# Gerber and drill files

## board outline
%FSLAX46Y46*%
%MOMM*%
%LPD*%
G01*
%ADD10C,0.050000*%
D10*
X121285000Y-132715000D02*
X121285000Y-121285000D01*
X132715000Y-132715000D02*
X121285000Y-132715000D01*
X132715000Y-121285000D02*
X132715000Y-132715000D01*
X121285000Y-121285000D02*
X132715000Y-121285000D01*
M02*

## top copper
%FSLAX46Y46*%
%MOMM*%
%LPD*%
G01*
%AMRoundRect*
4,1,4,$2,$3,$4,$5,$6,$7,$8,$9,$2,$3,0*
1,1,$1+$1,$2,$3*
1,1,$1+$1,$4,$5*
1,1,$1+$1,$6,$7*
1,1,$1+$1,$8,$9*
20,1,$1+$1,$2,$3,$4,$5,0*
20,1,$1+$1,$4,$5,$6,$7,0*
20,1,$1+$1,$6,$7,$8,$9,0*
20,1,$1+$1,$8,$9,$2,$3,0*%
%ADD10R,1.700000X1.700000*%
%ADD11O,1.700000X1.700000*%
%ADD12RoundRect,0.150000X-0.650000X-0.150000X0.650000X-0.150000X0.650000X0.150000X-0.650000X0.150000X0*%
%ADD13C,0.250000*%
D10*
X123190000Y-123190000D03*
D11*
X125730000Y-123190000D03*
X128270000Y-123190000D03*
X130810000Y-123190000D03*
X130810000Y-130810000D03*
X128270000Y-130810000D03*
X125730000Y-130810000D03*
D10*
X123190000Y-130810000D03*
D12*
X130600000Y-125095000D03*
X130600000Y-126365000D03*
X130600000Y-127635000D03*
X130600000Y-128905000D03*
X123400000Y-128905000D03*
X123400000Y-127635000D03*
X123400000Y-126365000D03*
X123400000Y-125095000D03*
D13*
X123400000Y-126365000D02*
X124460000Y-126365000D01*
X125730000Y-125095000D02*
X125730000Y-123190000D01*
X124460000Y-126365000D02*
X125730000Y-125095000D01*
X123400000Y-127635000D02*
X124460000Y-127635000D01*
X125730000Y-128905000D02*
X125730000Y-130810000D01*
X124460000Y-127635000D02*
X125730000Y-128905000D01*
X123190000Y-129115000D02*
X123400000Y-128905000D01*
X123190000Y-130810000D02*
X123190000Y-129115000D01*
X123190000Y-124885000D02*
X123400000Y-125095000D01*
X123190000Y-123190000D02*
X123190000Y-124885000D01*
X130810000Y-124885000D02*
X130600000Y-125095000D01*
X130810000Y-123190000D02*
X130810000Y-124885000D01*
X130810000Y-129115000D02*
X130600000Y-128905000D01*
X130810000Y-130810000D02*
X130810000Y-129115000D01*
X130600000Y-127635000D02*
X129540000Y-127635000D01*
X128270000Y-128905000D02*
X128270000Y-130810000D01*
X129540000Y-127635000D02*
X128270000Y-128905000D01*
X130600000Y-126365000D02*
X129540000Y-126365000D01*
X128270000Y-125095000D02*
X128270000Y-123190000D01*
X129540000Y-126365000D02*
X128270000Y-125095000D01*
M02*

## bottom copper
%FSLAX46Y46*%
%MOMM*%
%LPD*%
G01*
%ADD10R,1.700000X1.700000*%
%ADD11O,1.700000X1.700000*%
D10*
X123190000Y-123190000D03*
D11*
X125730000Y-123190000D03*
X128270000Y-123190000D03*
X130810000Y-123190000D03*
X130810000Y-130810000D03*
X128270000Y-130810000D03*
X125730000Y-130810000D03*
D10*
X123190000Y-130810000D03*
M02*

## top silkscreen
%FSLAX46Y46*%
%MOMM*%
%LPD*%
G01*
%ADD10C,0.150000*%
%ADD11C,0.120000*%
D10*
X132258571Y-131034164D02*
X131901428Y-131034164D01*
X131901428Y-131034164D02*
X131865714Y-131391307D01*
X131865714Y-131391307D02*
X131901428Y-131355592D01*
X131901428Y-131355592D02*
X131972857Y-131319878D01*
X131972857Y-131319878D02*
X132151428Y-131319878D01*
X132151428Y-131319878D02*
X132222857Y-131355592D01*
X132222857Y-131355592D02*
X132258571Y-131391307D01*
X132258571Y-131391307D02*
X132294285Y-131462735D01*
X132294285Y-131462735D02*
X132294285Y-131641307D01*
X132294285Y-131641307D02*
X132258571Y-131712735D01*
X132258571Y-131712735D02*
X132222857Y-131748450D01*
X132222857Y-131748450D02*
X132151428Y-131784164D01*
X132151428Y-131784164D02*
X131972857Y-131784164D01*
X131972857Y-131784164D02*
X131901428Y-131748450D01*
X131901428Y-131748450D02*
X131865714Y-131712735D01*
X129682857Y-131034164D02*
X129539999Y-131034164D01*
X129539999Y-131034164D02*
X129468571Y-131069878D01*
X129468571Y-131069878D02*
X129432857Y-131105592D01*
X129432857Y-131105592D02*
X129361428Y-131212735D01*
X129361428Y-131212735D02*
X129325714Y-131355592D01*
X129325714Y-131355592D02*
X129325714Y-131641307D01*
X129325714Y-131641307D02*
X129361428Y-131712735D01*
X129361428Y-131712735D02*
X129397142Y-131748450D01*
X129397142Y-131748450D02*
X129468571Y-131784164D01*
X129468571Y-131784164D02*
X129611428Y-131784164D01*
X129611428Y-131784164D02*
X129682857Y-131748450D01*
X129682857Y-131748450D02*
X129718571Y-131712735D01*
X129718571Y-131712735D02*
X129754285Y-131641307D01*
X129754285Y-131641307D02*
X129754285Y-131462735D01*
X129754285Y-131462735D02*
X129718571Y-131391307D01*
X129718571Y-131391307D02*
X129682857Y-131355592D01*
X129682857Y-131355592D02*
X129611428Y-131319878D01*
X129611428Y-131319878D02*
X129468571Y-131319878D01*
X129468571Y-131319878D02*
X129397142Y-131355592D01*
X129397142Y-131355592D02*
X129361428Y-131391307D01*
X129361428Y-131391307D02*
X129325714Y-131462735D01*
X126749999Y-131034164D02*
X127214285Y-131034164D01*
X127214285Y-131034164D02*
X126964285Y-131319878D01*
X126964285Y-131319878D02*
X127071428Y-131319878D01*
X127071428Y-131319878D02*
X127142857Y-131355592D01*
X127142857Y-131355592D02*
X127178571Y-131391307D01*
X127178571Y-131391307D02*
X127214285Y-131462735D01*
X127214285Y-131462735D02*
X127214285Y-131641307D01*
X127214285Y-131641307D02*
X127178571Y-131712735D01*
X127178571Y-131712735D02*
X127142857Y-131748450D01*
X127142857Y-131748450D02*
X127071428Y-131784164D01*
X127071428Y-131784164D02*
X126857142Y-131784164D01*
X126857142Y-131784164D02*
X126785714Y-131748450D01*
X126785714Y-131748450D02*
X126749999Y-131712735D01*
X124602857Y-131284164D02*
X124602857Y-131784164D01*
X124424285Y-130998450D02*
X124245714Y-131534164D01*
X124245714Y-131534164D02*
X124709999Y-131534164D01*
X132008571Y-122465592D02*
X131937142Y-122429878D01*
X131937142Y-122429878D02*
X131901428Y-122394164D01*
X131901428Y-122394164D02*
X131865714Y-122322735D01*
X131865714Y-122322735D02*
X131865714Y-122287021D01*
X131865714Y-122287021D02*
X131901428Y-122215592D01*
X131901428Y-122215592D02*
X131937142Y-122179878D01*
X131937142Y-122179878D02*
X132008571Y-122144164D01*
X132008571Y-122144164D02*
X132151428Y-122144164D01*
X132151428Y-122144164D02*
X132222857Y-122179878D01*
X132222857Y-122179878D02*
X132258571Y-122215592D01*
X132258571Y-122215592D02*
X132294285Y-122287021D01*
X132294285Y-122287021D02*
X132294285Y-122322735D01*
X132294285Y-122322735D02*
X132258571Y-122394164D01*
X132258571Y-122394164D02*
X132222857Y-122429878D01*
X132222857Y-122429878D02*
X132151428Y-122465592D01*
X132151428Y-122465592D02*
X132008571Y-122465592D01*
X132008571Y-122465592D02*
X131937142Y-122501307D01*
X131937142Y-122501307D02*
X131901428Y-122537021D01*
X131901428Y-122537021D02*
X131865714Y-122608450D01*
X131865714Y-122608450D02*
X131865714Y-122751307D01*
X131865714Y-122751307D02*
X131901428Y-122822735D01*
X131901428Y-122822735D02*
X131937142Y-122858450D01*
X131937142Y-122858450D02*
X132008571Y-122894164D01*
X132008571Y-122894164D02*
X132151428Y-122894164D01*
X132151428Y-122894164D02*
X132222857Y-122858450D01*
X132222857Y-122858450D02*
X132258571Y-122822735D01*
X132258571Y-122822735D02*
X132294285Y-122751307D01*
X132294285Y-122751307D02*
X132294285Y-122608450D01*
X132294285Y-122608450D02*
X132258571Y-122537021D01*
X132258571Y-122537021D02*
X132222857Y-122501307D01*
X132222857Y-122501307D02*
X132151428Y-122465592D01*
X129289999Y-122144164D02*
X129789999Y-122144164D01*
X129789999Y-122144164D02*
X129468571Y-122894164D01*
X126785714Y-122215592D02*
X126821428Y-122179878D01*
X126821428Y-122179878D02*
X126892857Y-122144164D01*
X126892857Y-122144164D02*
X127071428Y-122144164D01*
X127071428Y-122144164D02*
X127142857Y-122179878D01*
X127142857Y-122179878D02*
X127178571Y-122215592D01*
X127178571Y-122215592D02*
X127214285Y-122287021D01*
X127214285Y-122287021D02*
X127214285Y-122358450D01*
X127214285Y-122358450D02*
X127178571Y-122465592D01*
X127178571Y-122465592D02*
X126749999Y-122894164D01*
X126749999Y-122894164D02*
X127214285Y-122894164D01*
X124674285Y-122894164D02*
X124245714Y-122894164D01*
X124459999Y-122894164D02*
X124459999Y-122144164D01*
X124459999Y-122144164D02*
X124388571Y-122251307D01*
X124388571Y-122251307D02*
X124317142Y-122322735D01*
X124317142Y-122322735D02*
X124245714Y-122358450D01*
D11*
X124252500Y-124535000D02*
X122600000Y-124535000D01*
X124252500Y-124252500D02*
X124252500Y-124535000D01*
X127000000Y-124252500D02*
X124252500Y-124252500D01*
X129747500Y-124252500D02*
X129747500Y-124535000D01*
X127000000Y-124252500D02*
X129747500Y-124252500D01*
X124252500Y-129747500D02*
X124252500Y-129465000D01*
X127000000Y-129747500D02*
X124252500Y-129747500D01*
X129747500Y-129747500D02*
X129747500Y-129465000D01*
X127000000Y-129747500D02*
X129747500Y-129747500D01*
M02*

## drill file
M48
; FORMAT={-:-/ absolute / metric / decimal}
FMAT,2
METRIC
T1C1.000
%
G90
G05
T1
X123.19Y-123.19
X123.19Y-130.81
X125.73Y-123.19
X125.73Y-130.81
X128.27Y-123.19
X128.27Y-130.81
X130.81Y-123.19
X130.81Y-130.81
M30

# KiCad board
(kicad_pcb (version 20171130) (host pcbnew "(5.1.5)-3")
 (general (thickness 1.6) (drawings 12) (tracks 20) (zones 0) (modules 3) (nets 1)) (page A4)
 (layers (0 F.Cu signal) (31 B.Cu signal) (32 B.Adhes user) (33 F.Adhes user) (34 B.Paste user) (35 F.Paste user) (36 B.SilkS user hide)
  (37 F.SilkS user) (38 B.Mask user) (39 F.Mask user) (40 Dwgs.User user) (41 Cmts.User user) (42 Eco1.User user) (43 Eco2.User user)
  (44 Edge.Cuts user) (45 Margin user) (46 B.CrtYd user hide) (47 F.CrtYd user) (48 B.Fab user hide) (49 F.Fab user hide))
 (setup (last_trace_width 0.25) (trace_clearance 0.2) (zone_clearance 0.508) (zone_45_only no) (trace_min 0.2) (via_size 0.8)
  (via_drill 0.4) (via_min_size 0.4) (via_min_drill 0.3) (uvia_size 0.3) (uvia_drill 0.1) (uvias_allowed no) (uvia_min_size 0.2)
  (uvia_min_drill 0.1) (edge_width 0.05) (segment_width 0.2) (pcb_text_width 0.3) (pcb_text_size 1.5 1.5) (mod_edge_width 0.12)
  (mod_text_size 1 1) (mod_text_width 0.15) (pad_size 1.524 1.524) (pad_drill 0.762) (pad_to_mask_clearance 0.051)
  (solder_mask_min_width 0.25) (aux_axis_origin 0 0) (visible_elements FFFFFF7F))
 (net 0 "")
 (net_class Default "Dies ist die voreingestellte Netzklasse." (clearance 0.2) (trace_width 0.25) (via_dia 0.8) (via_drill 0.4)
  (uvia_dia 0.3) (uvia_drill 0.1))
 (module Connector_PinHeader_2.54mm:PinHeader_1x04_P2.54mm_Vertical (layer B.Cu) (at 123.19 123.19 270)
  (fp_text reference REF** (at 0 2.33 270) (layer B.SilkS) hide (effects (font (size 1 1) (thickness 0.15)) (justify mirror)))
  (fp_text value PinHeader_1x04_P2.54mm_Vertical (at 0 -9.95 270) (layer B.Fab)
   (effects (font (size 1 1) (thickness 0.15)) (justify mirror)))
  (pad 1 thru_hole rect (at 0 0 270) (size 1.7 1.7) (drill 1) (layers *.Cu *.Mask))
  (pad 2 thru_hole oval (at 0 -2.54 270) (size 1.7 1.7) (drill 1) (layers *.Cu *.Mask))
  (pad 3 thru_hole oval (at 0 -5.08 270) (size 1.7 1.7) (drill 1) (layers *.Cu *.Mask))
  (pad 4 thru_hole oval (at 0 -7.62 270) (size 1.7 1.7) (drill 1) (layers *.Cu *.Mask)))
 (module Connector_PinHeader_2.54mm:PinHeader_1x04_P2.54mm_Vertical (layer B.Cu) (at 123.19 130.81 270)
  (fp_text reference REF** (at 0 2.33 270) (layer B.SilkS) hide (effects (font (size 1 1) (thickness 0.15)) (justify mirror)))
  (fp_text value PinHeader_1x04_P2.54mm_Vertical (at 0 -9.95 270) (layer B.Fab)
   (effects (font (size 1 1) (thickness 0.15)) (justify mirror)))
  (pad 4 thru_hole oval (at 0 -7.62 270) (size 1.7 1.7) (drill 1) (layers *.Cu *.Mask))
  (pad 3 thru_hole oval (at 0 -5.08 270) (size 1.7 1.7) (drill 1) (layers *.Cu *.Mask))
  (pad 2 thru_hole oval (at 0 -2.54 270) (size 1.7 1.7) (drill 1) (layers *.Cu *.Mask))
  (pad 1 thru_hole rect (at 0 0 270) (size 1.7 1.7) (drill 1) (layers *.Cu *.Mask)))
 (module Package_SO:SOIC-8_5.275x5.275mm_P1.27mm (layer F.Cu) (at 127 127)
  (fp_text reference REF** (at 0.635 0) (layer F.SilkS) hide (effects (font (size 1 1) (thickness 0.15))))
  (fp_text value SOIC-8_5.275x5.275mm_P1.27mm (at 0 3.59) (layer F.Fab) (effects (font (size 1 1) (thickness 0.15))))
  (fp_line (start -2.7475 -2.465) (end -4.4 -2.465) (layer F.SilkS) (width 0.12))
  (fp_line (start -2.7475 -2.7475) (end -2.7475 -2.465) (layer F.SilkS) (width 0.12))
  (fp_line (start 0 -2.7475) (end -2.7475 -2.7475) (layer F.SilkS) (width 0.12))
  (fp_line (start 2.7475 -2.7475) (end 2.7475 -2.465) (layer F.SilkS) (width 0.12))
  (fp_line (start 0 -2.7475) (end 2.7475 -2.7475) (layer F.SilkS) (width 0.12))
  (fp_line (start -2.7475 2.7475) (end -2.7475 2.465) (layer F.SilkS) (width 0.12))
  (fp_line (start 0 2.7475) (end -2.7475 2.7475) (layer F.SilkS) (width 0.12))
  (fp_line (start 2.7475 2.7475) (end 2.7475 2.465) (layer F.SilkS) (width 0.12))
  (fp_line (start 0 2.7475) (end 2.7475 2.7475) (layer F.SilkS) (width 0.12))
  (pad 8 smd roundrect (at 3.6 -1.905) (size 1.6 0.6) (layers F.Cu F.Paste F.Mask) (roundrect_rratio 0.25))
  (pad 7 smd roundrect (at 3.6 -0.635) (size 1.6 0.6) (layers F.Cu F.Paste F.Mask) (roundrect_rratio 0.25))
  (pad 6 smd roundrect (at 3.6 0.635) (size 1.6 0.6) (layers F.Cu F.Paste F.Mask) (roundrect_rratio 0.25))
  (pad 5 smd roundrect (at 3.6 1.905) (size 1.6 0.6) (layers F.Cu F.Paste F.Mask) (roundrect_rratio 0.25))
  (pad 4 smd roundrect (at -3.6 1.905) (size 1.6 0.6) (layers F.Cu F.Paste F.Mask) (roundrect_rratio 0.25))
  (pad 3 smd roundrect (at -3.6 0.635) (size 1.6 0.6) (layers F.Cu F.Paste F.Mask) (roundrect_rratio 0.25))
  (pad 2 smd roundrect (at -3.6 -0.635) (size 1.6 0.6) (layers F.Cu F.Paste F.Mask) (roundrect_rratio 0.25))
  (pad 1 smd roundrect (at -3.6 -1.905) (size 1.6 0.6) (layers F.Cu F.Paste F.Mask) (roundrect_rratio 0.25)))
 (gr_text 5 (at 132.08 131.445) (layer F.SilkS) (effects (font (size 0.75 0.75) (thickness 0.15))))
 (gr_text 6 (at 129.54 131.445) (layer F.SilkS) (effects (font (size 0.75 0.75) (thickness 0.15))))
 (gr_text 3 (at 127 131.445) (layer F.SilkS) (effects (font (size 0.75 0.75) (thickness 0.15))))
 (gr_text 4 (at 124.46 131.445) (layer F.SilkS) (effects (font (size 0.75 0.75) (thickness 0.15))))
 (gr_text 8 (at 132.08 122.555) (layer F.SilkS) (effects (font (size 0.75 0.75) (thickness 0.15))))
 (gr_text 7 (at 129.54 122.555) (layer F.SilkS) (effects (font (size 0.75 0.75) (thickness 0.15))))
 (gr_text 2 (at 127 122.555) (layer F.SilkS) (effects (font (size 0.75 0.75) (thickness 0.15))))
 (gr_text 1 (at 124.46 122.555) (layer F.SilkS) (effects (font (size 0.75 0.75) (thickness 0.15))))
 (gr_line (start 121.285 132.715) (end 121.285 121.285) (layer Edge.Cuts) (width 0.05))
 (gr_line (start 132.715 132.715) (end 121.285 132.715) (layer Edge.Cuts) (width 0.05))
 (gr_line (start 132.715 121.285) (end 132.715 132.715) (layer Edge.Cuts) (width 0.05))
 (gr_line (start 121.285 121.285) (end 132.715 121.285) (layer Edge.Cuts) (width 0.05))
 (segment (start 123.4 126.365) (end 124.46 126.365) (width 0.25) (layer F.Cu) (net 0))
 (segment (start 125.73 125.095) (end 125.73 123.19) (width 0.25) (layer F.Cu) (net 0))
 (segment (start 124.46 126.365) (end 125.73 125.095) (width 0.25) (layer F.Cu) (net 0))
 (segment (start 123.4 127.635) (end 124.46 127.635) (width 0.25) (layer F.Cu) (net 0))
 (segment (start 125.73 128.905) (end 125.73 130.81) (width 0.25) (layer F.Cu) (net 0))
 (segment (start 124.46 127.635) (end 125.73 128.905) (width 0.25) (layer F.Cu) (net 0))
 (segment (start 123.19 129.115) (end 123.4 128.905) (width 0.25) (layer F.Cu) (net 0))
 (segment (start 123.19 130.81) (end 123.19 129.115) (width 0.25) (layer F.Cu) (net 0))
 (segment (start 123.19 124.885) (end 123.4 125.095) (width 0.25) (layer F.Cu) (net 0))
 (segment (start 123.19 123.19) (end 123.19 124.885) (width 0.25) (layer F.Cu) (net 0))
 (segment (start 130.81 124.885) (end 130.6 125.095) (width 0.25) (layer F.Cu) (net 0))
 (segment (start 130.81 123.19) (end 130.81 124.885) (width 0.25) (layer F.Cu) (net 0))
 (segment (start 130.81 129.115) (end 130.6 128.905) (width 0.25) (layer F.Cu) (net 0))
 (segment (start 130.81 130.81) (end 130.81 129.115) (width 0.25) (layer F.Cu) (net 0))
 (segment (start 130.6 127.635) (end 129.54 127.635) (width 0.25) (layer F.Cu) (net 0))
 (segment (start 128.27 128.905) (end 128.27 130.81) (width 0.25) (layer F.Cu) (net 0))
 (segment (start 129.54 127.635) (end 128.27 128.905) (width 0.25) (layer F.Cu) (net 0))
 (segment (start 130.6 126.365) (end 129.54 126.365) (width 0.25) (layer F.Cu) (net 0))
 (segment (start 128.27 125.095) (end 128.27 123.19) (width 0.25) (layer F.Cu) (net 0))
 (segment (start 129.54 126.365) (end 128.27 125.095) (width 0.25) (layer F.Cu) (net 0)))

